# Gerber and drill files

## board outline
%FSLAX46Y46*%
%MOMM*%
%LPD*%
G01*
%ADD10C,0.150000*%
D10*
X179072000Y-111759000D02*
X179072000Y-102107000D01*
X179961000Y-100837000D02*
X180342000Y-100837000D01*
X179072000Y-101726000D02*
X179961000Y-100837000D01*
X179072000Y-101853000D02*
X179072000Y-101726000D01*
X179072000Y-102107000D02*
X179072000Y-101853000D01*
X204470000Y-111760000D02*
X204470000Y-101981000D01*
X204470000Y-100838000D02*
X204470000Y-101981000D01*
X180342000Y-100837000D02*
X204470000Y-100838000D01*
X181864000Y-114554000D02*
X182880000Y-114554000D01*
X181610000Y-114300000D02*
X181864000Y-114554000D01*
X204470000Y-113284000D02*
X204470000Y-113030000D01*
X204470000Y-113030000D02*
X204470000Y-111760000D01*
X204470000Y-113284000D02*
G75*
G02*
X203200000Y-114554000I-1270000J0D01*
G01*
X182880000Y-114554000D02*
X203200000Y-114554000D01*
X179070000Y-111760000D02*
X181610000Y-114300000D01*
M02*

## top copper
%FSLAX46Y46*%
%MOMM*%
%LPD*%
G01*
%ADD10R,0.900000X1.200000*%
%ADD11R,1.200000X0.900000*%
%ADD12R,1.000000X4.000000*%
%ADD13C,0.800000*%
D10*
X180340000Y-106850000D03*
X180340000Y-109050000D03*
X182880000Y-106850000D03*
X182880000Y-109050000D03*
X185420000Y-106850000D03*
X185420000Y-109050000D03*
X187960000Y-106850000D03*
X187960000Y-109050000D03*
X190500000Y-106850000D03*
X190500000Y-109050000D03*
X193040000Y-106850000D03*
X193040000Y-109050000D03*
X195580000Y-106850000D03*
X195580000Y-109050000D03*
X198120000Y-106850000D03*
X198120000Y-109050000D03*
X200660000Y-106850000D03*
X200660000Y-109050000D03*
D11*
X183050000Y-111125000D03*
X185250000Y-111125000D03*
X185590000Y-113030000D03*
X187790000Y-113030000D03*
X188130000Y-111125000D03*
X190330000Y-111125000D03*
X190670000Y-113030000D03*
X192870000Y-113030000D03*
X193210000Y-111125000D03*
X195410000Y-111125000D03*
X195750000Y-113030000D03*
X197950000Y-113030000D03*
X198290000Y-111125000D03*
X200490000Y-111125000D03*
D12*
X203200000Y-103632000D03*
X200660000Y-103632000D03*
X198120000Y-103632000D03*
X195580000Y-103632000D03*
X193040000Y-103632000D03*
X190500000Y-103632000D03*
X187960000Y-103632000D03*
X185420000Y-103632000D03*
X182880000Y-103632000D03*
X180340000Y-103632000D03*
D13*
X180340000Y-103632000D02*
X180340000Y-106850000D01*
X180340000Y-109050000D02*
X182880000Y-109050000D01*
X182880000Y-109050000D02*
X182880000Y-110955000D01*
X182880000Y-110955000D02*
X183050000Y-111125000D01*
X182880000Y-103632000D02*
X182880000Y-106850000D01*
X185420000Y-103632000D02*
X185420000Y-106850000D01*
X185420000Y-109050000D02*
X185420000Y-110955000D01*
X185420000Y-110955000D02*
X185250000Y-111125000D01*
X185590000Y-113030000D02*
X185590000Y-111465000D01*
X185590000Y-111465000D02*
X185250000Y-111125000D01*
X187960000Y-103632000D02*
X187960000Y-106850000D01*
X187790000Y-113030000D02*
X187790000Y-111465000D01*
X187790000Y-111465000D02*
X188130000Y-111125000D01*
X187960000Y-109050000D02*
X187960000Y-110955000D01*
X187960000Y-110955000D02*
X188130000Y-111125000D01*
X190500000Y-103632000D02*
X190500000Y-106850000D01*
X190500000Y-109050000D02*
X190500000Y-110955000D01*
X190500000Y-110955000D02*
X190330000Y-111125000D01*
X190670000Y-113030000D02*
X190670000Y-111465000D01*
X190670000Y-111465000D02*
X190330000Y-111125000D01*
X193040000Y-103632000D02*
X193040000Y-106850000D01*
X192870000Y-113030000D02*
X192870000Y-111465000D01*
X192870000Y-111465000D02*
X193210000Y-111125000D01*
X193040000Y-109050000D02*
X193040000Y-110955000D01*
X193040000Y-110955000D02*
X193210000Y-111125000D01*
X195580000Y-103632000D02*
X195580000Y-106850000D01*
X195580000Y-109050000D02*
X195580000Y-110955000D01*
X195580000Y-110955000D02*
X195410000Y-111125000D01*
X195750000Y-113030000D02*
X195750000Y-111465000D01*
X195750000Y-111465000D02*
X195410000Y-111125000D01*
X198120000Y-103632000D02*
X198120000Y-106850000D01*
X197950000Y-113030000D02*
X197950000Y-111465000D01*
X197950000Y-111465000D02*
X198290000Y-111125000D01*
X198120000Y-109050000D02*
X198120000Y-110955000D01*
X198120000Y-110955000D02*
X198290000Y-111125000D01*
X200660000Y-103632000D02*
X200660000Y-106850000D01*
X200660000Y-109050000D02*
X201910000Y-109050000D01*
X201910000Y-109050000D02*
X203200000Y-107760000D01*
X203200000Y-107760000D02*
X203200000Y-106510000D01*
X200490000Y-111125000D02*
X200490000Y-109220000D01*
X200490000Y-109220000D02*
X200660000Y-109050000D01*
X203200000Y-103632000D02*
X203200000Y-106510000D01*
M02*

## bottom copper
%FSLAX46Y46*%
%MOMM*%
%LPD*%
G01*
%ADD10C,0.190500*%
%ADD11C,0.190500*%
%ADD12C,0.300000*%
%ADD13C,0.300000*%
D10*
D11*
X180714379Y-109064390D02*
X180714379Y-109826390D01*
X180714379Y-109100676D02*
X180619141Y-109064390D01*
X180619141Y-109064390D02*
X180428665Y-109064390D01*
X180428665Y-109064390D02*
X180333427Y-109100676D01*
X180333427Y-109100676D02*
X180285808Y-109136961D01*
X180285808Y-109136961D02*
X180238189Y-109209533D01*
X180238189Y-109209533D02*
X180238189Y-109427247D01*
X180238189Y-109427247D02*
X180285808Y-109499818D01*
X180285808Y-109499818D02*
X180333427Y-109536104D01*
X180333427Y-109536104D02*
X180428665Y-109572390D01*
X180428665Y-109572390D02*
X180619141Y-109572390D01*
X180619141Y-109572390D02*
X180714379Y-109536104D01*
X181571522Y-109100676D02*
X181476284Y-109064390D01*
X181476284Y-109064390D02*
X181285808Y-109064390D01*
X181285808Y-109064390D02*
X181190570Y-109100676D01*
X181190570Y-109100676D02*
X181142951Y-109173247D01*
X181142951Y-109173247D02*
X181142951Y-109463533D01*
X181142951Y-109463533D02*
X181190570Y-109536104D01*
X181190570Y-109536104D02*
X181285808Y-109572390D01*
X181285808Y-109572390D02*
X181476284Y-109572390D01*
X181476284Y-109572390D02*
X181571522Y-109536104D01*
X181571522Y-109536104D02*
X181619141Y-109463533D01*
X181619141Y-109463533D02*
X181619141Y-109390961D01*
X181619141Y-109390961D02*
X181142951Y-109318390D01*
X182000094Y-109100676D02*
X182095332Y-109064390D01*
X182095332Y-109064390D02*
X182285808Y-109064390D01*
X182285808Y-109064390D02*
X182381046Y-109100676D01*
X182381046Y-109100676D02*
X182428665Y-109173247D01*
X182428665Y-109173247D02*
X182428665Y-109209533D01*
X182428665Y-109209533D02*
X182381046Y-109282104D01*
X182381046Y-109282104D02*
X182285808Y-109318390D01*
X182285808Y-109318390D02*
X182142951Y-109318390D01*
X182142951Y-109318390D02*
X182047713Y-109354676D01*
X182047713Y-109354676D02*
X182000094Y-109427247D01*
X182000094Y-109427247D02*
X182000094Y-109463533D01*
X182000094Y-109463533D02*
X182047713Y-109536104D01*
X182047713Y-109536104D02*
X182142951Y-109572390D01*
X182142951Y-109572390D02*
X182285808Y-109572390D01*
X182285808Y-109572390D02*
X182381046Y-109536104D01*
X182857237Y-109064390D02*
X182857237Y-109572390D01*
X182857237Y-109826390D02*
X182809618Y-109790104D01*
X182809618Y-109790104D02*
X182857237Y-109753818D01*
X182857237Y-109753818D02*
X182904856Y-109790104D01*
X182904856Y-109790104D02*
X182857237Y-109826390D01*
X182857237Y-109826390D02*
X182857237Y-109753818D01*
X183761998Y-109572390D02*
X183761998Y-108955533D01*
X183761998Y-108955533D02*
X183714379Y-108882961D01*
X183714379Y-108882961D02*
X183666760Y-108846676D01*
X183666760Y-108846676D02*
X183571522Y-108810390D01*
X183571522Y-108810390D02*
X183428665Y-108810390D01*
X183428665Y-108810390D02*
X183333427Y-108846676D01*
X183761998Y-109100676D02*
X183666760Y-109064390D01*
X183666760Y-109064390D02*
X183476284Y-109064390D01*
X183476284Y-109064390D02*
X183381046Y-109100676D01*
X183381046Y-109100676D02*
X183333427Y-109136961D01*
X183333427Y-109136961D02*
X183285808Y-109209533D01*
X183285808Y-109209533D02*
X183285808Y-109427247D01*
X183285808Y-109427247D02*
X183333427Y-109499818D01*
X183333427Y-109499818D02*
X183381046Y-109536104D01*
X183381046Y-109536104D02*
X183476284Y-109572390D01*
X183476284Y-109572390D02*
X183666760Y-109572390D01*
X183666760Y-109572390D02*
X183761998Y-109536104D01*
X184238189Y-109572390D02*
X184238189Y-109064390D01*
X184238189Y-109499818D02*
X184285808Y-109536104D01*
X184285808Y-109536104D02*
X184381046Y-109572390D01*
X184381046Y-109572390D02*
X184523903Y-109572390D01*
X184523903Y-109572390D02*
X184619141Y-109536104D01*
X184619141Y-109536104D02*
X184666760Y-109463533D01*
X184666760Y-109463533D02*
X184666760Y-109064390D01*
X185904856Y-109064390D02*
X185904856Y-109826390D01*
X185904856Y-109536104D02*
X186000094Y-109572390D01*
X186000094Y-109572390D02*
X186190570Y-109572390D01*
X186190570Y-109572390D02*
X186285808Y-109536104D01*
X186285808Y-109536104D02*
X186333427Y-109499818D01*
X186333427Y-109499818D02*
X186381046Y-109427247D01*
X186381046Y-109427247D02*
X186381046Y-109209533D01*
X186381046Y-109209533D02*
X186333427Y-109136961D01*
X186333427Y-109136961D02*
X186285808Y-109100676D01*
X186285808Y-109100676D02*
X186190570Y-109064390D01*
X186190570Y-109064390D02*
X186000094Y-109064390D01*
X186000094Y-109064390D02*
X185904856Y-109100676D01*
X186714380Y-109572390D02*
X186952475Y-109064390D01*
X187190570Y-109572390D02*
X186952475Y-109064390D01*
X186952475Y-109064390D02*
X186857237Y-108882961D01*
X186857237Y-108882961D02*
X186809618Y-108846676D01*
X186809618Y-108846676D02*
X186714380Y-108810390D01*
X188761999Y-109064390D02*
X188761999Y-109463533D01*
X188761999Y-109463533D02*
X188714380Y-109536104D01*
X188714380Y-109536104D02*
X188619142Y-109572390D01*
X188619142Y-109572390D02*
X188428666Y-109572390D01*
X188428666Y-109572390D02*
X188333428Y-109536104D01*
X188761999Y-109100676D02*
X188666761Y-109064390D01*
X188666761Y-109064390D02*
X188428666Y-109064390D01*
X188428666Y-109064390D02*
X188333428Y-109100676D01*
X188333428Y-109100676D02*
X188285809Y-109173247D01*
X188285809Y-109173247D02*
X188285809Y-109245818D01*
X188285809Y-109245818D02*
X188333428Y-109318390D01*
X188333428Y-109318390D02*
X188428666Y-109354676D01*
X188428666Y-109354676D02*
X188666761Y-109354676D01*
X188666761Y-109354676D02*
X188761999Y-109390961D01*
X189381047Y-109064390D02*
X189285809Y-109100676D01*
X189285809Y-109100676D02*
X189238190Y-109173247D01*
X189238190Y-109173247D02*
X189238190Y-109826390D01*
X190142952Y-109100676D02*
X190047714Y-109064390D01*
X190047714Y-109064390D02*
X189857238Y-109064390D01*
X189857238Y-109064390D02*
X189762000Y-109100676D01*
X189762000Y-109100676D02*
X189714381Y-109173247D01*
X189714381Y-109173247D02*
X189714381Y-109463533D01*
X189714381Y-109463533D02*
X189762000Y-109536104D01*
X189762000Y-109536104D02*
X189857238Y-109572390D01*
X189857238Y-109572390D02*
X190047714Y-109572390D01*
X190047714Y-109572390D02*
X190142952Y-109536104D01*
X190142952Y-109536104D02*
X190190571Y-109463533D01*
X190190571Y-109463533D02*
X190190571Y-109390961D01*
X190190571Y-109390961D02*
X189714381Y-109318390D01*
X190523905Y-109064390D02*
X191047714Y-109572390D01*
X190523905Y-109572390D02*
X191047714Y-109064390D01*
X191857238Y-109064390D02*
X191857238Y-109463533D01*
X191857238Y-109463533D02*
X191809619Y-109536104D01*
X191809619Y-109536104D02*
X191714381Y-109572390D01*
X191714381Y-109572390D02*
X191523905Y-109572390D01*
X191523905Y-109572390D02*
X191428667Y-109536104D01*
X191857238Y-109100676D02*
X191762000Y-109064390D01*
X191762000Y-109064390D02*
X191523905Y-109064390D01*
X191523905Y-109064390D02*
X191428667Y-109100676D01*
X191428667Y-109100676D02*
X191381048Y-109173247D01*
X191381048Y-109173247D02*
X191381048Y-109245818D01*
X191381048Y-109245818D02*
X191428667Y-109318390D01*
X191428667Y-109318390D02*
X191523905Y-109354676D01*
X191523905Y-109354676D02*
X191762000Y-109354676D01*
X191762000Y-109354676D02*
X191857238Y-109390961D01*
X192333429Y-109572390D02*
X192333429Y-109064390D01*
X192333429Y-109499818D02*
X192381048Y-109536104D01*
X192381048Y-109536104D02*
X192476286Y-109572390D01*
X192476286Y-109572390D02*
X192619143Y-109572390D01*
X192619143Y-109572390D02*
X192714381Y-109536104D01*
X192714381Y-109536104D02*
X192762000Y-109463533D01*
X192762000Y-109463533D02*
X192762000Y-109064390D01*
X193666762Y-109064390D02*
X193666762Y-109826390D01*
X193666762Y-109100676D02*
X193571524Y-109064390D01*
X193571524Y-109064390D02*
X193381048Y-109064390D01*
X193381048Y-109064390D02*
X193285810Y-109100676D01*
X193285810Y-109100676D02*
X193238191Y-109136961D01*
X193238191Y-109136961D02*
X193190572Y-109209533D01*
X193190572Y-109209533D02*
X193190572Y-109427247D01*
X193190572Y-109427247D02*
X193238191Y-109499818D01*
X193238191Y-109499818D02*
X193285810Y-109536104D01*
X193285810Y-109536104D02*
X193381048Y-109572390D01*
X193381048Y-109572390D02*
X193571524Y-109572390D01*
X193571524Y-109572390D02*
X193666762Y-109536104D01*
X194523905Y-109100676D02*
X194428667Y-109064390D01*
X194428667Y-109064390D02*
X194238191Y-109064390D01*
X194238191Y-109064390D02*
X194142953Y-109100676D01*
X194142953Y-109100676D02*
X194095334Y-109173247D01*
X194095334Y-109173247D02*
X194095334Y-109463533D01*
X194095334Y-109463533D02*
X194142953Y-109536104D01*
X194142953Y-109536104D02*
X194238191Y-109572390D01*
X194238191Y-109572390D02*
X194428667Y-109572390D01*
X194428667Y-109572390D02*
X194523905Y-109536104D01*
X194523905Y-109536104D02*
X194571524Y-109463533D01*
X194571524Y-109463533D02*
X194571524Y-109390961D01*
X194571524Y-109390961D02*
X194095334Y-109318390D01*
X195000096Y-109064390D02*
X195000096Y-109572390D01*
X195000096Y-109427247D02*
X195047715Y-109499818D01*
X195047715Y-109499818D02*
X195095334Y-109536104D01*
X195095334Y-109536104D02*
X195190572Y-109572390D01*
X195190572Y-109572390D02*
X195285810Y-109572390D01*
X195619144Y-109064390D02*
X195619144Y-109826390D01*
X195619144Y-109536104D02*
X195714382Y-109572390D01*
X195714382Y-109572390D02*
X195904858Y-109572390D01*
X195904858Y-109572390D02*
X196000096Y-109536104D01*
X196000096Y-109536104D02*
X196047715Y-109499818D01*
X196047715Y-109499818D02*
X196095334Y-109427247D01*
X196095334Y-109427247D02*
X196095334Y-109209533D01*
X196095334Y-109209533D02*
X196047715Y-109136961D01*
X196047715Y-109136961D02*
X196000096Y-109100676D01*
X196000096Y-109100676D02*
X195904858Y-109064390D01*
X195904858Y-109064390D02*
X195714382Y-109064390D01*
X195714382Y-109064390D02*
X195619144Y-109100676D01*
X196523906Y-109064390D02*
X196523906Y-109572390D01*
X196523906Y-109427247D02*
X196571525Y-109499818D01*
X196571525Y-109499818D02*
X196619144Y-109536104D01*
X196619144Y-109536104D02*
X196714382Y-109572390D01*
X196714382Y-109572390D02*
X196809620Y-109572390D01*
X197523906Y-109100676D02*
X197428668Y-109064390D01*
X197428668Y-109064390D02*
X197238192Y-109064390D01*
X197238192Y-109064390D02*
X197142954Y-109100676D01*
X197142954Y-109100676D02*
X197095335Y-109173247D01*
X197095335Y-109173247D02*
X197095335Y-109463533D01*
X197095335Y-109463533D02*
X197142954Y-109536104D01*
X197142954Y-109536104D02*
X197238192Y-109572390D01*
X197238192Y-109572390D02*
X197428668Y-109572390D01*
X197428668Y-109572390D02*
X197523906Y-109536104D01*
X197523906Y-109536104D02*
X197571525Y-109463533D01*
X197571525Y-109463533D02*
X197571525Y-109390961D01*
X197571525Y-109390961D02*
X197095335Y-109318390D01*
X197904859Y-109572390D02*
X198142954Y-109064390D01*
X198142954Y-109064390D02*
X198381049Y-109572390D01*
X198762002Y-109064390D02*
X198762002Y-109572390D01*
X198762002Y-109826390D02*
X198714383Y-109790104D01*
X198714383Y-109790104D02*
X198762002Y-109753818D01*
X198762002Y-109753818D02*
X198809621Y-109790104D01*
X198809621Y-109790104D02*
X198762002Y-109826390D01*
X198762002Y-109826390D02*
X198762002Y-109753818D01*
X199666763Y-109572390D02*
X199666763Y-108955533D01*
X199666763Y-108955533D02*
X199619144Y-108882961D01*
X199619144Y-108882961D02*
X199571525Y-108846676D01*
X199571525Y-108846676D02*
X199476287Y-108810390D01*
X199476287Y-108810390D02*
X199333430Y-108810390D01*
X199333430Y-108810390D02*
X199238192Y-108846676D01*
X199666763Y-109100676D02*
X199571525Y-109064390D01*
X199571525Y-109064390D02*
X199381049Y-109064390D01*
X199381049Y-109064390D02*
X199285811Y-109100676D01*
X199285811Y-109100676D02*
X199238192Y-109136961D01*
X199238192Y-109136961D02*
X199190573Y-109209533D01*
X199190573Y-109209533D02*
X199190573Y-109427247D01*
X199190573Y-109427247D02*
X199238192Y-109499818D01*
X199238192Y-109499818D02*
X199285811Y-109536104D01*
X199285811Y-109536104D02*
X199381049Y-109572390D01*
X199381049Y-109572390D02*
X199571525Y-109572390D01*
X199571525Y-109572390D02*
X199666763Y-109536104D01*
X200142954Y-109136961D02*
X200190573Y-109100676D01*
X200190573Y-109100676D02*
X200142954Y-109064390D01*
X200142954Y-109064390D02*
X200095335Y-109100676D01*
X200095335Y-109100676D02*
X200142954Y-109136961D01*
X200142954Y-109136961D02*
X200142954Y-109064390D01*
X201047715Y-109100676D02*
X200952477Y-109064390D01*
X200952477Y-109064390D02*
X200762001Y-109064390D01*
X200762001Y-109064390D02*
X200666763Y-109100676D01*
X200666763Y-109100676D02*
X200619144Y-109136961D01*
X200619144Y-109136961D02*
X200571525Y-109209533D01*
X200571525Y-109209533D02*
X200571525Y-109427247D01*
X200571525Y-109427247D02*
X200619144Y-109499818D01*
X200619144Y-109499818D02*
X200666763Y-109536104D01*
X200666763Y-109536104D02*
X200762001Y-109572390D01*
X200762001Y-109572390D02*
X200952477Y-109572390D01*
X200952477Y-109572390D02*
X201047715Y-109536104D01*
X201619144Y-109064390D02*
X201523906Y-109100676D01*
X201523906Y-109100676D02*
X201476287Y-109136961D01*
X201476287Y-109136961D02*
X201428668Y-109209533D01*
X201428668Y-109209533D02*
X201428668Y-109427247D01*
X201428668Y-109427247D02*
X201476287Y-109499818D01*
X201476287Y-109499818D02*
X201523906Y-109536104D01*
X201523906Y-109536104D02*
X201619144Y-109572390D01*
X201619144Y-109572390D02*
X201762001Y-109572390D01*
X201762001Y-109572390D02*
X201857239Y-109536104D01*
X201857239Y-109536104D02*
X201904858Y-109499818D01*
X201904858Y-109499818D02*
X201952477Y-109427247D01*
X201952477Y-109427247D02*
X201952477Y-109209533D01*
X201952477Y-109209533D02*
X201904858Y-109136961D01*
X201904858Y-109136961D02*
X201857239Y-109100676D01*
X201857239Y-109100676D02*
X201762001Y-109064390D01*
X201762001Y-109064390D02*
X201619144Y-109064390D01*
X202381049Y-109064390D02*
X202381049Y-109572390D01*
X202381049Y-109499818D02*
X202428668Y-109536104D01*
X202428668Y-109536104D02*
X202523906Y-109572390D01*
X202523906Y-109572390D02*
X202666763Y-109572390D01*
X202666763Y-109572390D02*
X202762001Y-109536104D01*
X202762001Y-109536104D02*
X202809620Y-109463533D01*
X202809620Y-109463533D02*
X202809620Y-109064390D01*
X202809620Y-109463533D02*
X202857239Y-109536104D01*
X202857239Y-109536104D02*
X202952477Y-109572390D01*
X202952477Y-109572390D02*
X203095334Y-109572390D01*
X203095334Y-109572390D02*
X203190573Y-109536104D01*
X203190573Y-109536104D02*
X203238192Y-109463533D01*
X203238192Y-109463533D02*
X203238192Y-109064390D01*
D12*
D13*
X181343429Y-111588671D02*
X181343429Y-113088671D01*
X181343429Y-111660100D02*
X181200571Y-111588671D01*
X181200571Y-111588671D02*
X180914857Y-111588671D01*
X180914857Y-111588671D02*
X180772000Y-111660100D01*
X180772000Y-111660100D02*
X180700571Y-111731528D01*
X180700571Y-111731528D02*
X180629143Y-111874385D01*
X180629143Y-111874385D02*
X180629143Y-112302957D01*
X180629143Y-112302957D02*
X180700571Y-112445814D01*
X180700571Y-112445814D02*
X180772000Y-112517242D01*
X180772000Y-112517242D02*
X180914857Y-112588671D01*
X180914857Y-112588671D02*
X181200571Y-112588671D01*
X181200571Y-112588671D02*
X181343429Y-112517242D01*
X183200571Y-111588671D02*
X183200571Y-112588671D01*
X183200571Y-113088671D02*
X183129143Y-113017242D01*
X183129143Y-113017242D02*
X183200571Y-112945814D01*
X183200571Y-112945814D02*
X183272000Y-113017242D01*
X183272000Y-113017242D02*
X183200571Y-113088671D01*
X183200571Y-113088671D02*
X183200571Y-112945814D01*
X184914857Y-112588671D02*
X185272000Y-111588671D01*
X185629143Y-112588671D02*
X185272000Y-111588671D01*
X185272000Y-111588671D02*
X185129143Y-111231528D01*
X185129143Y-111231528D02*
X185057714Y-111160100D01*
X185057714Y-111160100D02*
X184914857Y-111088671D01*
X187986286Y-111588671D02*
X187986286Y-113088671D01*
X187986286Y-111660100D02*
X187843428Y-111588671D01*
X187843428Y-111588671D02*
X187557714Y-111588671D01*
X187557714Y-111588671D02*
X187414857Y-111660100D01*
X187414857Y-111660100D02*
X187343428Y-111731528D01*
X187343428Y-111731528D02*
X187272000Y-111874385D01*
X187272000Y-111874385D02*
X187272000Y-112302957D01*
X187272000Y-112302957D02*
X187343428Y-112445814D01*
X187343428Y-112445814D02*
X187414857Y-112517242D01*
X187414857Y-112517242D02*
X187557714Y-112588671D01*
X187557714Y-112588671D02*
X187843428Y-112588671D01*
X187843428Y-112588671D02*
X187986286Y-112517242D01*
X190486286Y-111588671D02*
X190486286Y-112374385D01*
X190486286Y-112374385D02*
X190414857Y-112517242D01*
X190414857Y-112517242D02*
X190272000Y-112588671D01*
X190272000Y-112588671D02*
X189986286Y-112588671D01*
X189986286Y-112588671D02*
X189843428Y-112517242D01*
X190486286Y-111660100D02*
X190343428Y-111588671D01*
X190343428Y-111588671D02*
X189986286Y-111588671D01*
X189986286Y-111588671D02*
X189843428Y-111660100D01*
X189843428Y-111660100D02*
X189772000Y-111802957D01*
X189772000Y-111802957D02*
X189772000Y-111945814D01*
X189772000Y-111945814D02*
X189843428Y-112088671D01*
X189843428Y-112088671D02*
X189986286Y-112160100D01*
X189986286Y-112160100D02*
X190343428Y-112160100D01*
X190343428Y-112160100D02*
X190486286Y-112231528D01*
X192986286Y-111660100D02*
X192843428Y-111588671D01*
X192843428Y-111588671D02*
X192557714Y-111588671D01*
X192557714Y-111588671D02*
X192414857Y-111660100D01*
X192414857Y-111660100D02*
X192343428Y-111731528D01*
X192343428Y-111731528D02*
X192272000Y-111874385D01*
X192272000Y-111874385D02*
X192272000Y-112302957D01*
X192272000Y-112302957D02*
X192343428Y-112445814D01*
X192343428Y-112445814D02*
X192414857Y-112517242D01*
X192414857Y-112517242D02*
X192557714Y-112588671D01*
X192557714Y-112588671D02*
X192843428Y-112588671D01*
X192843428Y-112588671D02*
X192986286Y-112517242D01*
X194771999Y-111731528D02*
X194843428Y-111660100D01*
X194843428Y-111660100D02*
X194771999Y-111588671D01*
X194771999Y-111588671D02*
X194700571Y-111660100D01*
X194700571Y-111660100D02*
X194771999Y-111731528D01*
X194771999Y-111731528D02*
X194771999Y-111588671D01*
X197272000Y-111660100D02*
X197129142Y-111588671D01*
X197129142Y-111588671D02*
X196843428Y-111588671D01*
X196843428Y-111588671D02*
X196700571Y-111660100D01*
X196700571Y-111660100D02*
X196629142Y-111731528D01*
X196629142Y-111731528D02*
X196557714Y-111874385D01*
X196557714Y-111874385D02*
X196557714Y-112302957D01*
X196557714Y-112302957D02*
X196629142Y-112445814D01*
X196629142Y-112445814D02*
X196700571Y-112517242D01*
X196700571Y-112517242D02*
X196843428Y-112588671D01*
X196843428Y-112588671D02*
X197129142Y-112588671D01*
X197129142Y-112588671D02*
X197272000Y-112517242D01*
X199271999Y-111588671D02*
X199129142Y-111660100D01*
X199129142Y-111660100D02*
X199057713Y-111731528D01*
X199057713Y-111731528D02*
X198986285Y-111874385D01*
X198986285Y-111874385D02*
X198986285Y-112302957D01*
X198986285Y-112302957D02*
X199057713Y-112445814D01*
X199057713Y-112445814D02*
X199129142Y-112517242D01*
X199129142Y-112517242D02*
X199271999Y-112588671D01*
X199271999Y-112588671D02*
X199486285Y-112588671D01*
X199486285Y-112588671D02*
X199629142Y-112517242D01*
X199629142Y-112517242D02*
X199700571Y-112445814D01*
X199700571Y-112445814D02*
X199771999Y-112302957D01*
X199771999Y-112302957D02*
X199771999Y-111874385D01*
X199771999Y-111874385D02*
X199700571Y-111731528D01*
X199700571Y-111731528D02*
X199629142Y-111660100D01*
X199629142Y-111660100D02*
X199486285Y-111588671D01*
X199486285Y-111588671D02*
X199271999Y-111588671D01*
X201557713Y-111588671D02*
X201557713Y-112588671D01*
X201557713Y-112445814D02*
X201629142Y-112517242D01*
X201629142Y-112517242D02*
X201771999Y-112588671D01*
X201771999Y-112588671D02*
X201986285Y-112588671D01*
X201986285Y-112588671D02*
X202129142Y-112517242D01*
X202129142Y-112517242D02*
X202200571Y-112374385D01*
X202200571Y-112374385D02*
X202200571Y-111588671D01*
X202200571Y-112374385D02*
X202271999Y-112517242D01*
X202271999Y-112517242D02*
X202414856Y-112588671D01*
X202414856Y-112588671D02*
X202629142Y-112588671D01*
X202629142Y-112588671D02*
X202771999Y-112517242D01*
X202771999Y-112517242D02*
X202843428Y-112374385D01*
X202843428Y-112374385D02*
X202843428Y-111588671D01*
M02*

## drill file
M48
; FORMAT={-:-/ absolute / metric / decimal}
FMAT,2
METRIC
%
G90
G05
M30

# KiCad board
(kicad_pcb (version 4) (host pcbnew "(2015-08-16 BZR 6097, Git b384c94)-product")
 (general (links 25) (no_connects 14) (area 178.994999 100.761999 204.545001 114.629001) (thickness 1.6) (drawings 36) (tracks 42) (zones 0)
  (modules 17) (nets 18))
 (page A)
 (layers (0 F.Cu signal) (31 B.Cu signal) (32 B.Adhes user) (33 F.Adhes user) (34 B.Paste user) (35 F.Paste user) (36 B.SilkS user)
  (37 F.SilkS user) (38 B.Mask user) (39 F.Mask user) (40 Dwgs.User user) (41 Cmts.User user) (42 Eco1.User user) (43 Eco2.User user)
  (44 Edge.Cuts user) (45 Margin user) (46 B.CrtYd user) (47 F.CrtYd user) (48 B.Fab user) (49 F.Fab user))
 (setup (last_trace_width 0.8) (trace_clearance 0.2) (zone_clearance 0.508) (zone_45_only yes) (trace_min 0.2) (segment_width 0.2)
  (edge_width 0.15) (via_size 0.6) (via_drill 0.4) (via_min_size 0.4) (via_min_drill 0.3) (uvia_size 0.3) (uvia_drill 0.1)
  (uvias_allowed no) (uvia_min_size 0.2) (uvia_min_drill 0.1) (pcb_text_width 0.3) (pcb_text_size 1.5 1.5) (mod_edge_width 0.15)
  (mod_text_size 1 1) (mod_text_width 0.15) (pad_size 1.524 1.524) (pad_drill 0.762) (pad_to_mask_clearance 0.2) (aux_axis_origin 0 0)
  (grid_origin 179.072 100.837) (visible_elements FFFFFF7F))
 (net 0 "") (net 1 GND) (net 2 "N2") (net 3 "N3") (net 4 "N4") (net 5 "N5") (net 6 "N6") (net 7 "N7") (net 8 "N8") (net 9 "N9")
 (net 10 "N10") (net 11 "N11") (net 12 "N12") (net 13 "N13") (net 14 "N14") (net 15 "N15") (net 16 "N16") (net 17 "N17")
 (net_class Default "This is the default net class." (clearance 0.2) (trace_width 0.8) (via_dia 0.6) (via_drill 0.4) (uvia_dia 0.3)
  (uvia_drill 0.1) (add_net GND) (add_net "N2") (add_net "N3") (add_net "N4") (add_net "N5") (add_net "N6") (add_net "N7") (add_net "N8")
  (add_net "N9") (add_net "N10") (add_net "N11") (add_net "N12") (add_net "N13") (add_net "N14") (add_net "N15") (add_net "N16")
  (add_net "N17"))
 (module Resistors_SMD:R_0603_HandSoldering (layer F.Cu) (at 180.34 107.95 270)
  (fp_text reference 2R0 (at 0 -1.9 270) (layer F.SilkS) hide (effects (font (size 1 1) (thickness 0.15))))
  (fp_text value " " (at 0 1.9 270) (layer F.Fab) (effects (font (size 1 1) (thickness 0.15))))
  (pad 1 smd rect (at -1.1 0 270) (size 1.2 0.9) (layers F.Cu F.Paste F.Mask) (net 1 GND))
  (pad 2 smd rect (at 1.1 0 270) (size 1.2 0.9) (layers F.Cu F.Paste F.Mask) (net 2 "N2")))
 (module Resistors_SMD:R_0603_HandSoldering (layer F.Cu) (at 182.88 107.95 270)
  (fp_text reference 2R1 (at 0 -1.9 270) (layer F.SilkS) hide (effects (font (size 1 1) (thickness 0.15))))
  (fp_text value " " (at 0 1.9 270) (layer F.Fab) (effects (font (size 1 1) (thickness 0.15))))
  (pad 1 smd rect (at -1.1 0 270) (size 1.2 0.9) (layers F.Cu F.Paste F.Mask) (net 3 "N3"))
  (pad 2 smd rect (at 1.1 0 270) (size 1.2 0.9) (layers F.Cu F.Paste F.Mask) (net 2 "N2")))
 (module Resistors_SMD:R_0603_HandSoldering (layer F.Cu) (at 185.42 107.95 270)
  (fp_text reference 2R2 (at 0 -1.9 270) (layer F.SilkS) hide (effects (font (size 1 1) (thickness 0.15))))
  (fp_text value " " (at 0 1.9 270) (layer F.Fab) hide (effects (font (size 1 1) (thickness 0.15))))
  (pad 1 smd rect (at -1.1 0 270) (size 1.2 0.9) (layers F.Cu F.Paste F.Mask) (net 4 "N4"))
  (pad 2 smd rect (at 1.1 0 270) (size 1.2 0.9) (layers F.Cu F.Paste F.Mask) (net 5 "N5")))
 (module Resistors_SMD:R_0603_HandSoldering (layer F.Cu) (at 187.96 107.95 270)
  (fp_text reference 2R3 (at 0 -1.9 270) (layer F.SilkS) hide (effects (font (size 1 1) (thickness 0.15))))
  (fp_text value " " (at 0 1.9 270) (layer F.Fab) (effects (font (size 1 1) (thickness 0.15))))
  (pad 1 smd rect (at -1.1 0 270) (size 1.2 0.9) (layers F.Cu F.Paste F.Mask) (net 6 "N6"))
  (pad 2 smd rect (at 1.1 0 270) (size 1.2 0.9) (layers F.Cu F.Paste F.Mask) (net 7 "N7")))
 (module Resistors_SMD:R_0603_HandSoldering (layer F.Cu) (at 190.5 107.95 270)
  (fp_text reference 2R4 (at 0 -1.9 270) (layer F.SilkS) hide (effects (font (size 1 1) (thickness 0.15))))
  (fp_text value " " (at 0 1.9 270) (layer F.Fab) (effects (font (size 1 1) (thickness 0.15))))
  (pad 1 smd rect (at -1.1 0 270) (size 1.2 0.9) (layers F.Cu F.Paste F.Mask) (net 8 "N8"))
  (pad 2 smd rect (at 1.1 0 270) (size 1.2 0.9) (layers F.Cu F.Paste F.Mask) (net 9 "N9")))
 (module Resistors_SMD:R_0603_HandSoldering (layer F.Cu) (at 193.04 107.95 270)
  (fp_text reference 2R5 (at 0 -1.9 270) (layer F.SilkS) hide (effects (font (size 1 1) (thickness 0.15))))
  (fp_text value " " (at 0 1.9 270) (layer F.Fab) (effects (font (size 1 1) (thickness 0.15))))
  (pad 1 smd rect (at -1.1 0 270) (size 1.2 0.9) (layers F.Cu F.Paste F.Mask) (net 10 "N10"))
  (pad 2 smd rect (at 1.1 0 270) (size 1.2 0.9) (layers F.Cu F.Paste F.Mask) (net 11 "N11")))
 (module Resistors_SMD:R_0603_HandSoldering (layer F.Cu) (at 195.58 107.95 270)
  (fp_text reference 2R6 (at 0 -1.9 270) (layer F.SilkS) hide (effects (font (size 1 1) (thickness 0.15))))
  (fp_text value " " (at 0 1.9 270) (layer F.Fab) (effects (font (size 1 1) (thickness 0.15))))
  (pad 1 smd rect (at -1.1 0 270) (size 1.2 0.9) (layers F.Cu F.Paste F.Mask) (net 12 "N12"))
  (pad 2 smd rect (at 1.1 0 270) (size 1.2 0.9) (layers F.Cu F.Paste F.Mask) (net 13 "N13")))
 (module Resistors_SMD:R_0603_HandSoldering (layer F.Cu) (at 198.12 107.95 270)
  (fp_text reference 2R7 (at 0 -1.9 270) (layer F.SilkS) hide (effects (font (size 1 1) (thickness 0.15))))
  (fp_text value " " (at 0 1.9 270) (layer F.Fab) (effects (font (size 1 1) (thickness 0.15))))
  (pad 1 smd rect (at -1.1 0 270) (size 1.2 0.9) (layers F.Cu F.Paste F.Mask) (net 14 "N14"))
  (pad 2 smd rect (at 1.1 0 270) (size 1.2 0.9) (layers F.Cu F.Paste F.Mask) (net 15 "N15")))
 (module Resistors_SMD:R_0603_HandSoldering (layer F.Cu) (at 200.66 107.95 270)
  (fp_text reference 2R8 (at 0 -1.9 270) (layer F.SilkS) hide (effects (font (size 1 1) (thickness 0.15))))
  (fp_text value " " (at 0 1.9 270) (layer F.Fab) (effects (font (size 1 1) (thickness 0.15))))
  (pad 1 smd rect (at -1.1 0 270) (size 1.2 0.9) (layers F.Cu F.Paste F.Mask) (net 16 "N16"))
  (pad 2 smd rect (at 1.1 0 270) (size 1.2 0.9) (layers F.Cu F.Paste F.Mask) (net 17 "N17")))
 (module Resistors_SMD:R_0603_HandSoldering (layer F.Cu) (at 184.15 111.125)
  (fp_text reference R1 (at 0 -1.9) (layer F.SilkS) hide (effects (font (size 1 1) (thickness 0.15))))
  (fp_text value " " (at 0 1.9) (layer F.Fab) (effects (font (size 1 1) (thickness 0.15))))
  (pad 1 smd rect (at -1.1 0) (size 1.2 0.9) (layers F.Cu F.Paste F.Mask) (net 2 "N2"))
  (pad 2 smd rect (at 1.1 0) (size 1.2 0.9) (layers F.Cu F.Paste F.Mask) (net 5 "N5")))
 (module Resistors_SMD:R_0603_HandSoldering (layer F.Cu) (at 186.69 113.03)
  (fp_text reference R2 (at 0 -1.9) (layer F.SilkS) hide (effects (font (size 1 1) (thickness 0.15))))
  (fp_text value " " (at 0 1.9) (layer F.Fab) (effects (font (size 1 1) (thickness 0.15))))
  (pad 1 smd rect (at -1.1 0) (size 1.2 0.9) (layers F.Cu F.Paste F.Mask) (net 5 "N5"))
  (pad 2 smd rect (at 1.1 0) (size 1.2 0.9) (layers F.Cu F.Paste F.Mask) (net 7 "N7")))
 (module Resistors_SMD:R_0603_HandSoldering (layer F.Cu) (at 189.23 111.125)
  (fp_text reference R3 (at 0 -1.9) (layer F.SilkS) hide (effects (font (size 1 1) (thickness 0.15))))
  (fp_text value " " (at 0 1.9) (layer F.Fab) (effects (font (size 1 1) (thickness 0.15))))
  (pad 1 smd rect (at -1.1 0) (size 1.2 0.9) (layers F.Cu F.Paste F.Mask) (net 7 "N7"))
  (pad 2 smd rect (at 1.1 0) (size 1.2 0.9) (layers F.Cu F.Paste F.Mask) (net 9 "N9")))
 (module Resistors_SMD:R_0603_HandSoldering (layer F.Cu) (at 191.77 113.03)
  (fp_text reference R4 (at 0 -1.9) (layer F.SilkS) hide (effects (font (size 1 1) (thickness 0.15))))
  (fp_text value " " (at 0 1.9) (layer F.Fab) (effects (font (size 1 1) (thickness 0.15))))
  (pad 1 smd rect (at -1.1 0) (size 1.2 0.9) (layers F.Cu F.Paste F.Mask) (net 9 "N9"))
  (pad 2 smd rect (at 1.1 0) (size 1.2 0.9) (layers F.Cu F.Paste F.Mask) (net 11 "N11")))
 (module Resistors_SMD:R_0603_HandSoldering (layer F.Cu) (at 194.31 111.125)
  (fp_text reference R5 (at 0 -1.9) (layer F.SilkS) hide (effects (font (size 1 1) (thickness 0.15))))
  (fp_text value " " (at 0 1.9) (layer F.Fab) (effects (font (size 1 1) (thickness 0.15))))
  (pad 1 smd rect (at -1.1 0) (size 1.2 0.9) (layers F.Cu F.Paste F.Mask) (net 11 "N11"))
  (pad 2 smd rect (at 1.1 0) (size 1.2 0.9) (layers F.Cu F.Paste F.Mask) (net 13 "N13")))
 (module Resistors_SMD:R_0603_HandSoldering (layer F.Cu) (at 196.85 113.03)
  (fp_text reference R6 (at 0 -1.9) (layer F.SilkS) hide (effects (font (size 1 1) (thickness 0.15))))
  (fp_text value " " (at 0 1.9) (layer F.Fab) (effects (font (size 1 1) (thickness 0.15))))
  (pad 1 smd rect (at -1.1 0) (size 1.2 0.9) (layers F.Cu F.Paste F.Mask) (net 13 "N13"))
  (pad 2 smd rect (at 1.1 0) (size 1.2 0.9) (layers F.Cu F.Paste F.Mask) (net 15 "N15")))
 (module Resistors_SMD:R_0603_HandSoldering (layer F.Cu) (at 199.39 111.125)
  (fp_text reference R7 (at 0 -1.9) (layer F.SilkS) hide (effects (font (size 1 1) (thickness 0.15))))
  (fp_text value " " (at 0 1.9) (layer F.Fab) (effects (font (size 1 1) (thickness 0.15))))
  (pad 1 smd rect (at -1.1 0) (size 1.2 0.9) (layers F.Cu F.Paste F.Mask) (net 15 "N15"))
  (pad 2 smd rect (at 1.1 0) (size 1.2 0.9) (layers F.Cu F.Paste F.Mask) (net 17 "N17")))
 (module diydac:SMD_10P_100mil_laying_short (layer F.Cu) (at 180.34 103.632)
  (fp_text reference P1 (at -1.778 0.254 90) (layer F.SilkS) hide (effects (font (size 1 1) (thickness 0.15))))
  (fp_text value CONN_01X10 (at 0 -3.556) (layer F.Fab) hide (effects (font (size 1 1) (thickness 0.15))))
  (pad 10 smd rect (at 22.86 0) (size 1 4) (layers F.Cu F.Paste F.Mask) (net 17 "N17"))
  (pad 9 smd rect (at 20.32 0) (size 1 4) (layers F.Cu F.Paste F.Mask) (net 16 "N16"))
  (pad 8 smd rect (at 17.78 0) (size 1 4) (layers F.Cu F.Paste F.Mask) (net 14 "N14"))
  (pad 7 smd rect (at 15.24 0) (size 1 4) (layers F.Cu F.Paste F.Mask) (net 12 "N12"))
  (pad 6 smd rect (at 12.7 0) (size 1 4) (layers F.Cu F.Paste F.Mask) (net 10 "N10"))
  (pad 5 smd rect (at 10.16 0) (size 1 4) (layers F.Cu F.Paste F.Mask) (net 8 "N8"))
  (pad 4 smd rect (at 7.62 0) (size 1 4) (layers F.Cu F.Paste F.Mask) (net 6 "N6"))
  (pad 3 smd rect (at 5.08 0) (size 1 4) (layers F.Cu F.Paste F.Mask) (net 4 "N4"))
  (pad 2 smd rect (at 2.54 0) (size 1 4) (layers F.Cu F.Paste F.Mask) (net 3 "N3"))
  (pad 1 smd rect (at 0 0) (size 1 4) (layers F.Cu F.Paste F.Mask) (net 1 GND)))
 (gr_line (start 179.072 111.759) (end 179.072 102.107) (layer Edge.Cuts) (width 0.15))
 (gr_line (start 179.961 100.837) (end 180.342 100.837) (layer Edge.Cuts) (width 0.15))
 (gr_line (start 179.072 101.726) (end 179.961 100.837) (layer Edge.Cuts) (width 0.15))
 (gr_line (start 179.072 101.853) (end 179.072 101.726) (layer Edge.Cuts) (width 0.15))
 (gr_line (start 179.072 102.107) (end 179.072 101.853) (layer Edge.Cuts) (width 0.15))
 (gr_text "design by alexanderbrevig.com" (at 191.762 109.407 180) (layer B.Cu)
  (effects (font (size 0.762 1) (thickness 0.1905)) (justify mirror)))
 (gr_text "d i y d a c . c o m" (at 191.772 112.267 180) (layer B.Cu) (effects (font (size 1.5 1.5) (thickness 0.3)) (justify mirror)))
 (gr_line (start 204.47 111.76) (end 204.47 101.981) (angle 90) (layer Edge.Cuts) (width 0.15))
 (gr_line (start 204.47 100.838) (end 204.47 101.981) (angle 90) (layer Edge.Cuts) (width 0.15))
 (gr_line (start 180.342 100.837) (end 204.47 100.838) (angle 90) (layer Edge.Cuts) (width 0.15))
 (gr_line (start 181.864 114.554) (end 182.88 114.554) (angle 90) (layer Edge.Cuts) (width 0.15))
 (gr_line (start 181.61 114.3) (end 181.864 114.554) (angle 90) (layer Edge.Cuts) (width 0.15))
 (gr_line (start 204.47 113.284) (end 204.47 113.03) (angle 90) (layer Edge.Cuts) (width 0.15))
 (gr_line (start 204.47 113.03) (end 204.47 111.76) (angle 90) (layer Edge.Cuts) (width 0.15))
 (gr_arc (start 203.2 113.284) (end 204.47 113.284) (angle 90) (layer Edge.Cuts) (width 0.15))
 (gr_line (start 182.88 114.554) (end 203.2 114.554) (angle 90) (layer Edge.Cuts) (width 0.15))
 (gr_line (start 179.07 111.76) (end 181.61 114.3) (angle 90) (layer Edge.Cuts) (width 0.15))
 (segment (start 180.34 103.632) (end 180.34 106.85) (width 0.8) (layer F.Cu) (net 1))
 (segment (start 180.34 109.05) (end 182.88 109.05) (width 0.8) (layer F.Cu) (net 2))
 (segment (start 182.88 109.05) (end 182.88 110.955) (width 0.8) (layer F.Cu) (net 2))
 (segment (start 182.88 110.955) (end 183.05 111.125) (width 0.8) (layer F.Cu) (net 2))
 (segment (start 182.88 103.632) (end 182.88 106.85) (width 0.8) (layer F.Cu) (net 3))
 (segment (start 185.42 103.632) (end 185.42 106.85) (width 0.8) (layer F.Cu) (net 4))
 (segment (start 185.42 109.05) (end 185.42 110.955) (width 0.8) (layer F.Cu) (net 5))
 (segment (start 185.42 110.955) (end 185.25 111.125) (width 0.8) (layer F.Cu) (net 5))
 (segment (start 185.59 113.03) (end 185.59 111.465) (width 0.8) (layer F.Cu) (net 5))
 (segment (start 185.59 111.465) (end 185.25 111.125) (width 0.8) (layer F.Cu) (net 5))
 (segment (start 187.96 103.632) (end 187.96 106.85) (width 0.8) (layer F.Cu) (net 6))
 (segment (start 187.79 113.03) (end 187.79 111.465) (width 0.8) (layer F.Cu) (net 7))
 (segment (start 187.79 111.465) (end 188.13 111.125) (width 0.8) (layer F.Cu) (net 7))
 (segment (start 187.96 109.05) (end 187.96 110.955) (width 0.8) (layer F.Cu) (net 7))
 (segment (start 187.96 110.955) (end 188.13 111.125) (width 0.8) (layer F.Cu) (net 7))
 (segment (start 190.5 103.632) (end 190.5 106.85) (width 0.8) (layer F.Cu) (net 8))
 (segment (start 190.5 109.05) (end 190.5 110.955) (width 0.8) (layer F.Cu) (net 9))
 (segment (start 190.5 110.955) (end 190.33 111.125) (width 0.8) (layer F.Cu) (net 9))
 (segment (start 190.67 113.03) (end 190.67 111.465) (width 0.8) (layer F.Cu) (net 9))
 (segment (start 190.67 111.465) (end 190.33 111.125) (width 0.8) (layer F.Cu) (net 9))
 (segment (start 193.04 103.632) (end 193.04 106.85) (width 0.8) (layer F.Cu) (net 10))
 (segment (start 192.87 113.03) (end 192.87 111.465) (width 0.8) (layer F.Cu) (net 11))
 (segment (start 192.87 111.465) (end 193.21 111.125) (width 0.8) (layer F.Cu) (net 11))
 (segment (start 193.04 109.05) (end 193.04 110.955) (width 0.8) (layer F.Cu) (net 11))
 (segment (start 193.04 110.955) (end 193.21 111.125) (width 0.8) (layer F.Cu) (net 11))
 (segment (start 195.58 103.632) (end 195.58 106.85) (width 0.8) (layer F.Cu) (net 12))
 (segment (start 195.58 109.05) (end 195.58 110.955) (width 0.8) (layer F.Cu) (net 13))
 (segment (start 195.58 110.955) (end 195.41 111.125) (width 0.8) (layer F.Cu) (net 13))
 (segment (start 195.75 113.03) (end 195.75 111.465) (width 0.8) (layer F.Cu) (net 13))
 (segment (start 195.75 111.465) (end 195.41 111.125) (width 0.8) (layer F.Cu) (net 13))
 (segment (start 198.12 103.632) (end 198.12 106.85) (width 0.8) (layer F.Cu) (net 14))
 (segment (start 197.95 113.03) (end 197.95 111.465) (width 0.8) (layer F.Cu) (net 15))
 (segment (start 197.95 111.465) (end 198.29 111.125) (width 0.8) (layer F.Cu) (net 15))
 (segment (start 198.12 109.05) (end 198.12 110.955) (width 0.8) (layer F.Cu) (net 15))
 (segment (start 198.12 110.955) (end 198.29 111.125) (width 0.8) (layer F.Cu) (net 15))
 (segment (start 200.66 103.632) (end 200.66 106.85) (width 0.8) (layer F.Cu) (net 16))
 (segment (start 200.66 109.05) (end 201.91 109.05) (width 0.8) (layer F.Cu) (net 17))
 (segment (start 201.91 109.05) (end 203.2 107.76) (width 0.8) (layer F.Cu) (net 17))
 (segment (start 203.2 107.76) (end 203.2 106.51) (width 0.8) (layer F.Cu) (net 17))
 (segment (start 200.49 111.125) (end 200.49 109.22) (width 0.8) (layer F.Cu) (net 17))
 (segment (start 200.49 109.22) (end 200.66 109.05) (width 0.8) (layer F.Cu) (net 17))
 (segment (start 203.2 103.632) (end 203.2 106.51) (width 0.8) (layer F.Cu) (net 17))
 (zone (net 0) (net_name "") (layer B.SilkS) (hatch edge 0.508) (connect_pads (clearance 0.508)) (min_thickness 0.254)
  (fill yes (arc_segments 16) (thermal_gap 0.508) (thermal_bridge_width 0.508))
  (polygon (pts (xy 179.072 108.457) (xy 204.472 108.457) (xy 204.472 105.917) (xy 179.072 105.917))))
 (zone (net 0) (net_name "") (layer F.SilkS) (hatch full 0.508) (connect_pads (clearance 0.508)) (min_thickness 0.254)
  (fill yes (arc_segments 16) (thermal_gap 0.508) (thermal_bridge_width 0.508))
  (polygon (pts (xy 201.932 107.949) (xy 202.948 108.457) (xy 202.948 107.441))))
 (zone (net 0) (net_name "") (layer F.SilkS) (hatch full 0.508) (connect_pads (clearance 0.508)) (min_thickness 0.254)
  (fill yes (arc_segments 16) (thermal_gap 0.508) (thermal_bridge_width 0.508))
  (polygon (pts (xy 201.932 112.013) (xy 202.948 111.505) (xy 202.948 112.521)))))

